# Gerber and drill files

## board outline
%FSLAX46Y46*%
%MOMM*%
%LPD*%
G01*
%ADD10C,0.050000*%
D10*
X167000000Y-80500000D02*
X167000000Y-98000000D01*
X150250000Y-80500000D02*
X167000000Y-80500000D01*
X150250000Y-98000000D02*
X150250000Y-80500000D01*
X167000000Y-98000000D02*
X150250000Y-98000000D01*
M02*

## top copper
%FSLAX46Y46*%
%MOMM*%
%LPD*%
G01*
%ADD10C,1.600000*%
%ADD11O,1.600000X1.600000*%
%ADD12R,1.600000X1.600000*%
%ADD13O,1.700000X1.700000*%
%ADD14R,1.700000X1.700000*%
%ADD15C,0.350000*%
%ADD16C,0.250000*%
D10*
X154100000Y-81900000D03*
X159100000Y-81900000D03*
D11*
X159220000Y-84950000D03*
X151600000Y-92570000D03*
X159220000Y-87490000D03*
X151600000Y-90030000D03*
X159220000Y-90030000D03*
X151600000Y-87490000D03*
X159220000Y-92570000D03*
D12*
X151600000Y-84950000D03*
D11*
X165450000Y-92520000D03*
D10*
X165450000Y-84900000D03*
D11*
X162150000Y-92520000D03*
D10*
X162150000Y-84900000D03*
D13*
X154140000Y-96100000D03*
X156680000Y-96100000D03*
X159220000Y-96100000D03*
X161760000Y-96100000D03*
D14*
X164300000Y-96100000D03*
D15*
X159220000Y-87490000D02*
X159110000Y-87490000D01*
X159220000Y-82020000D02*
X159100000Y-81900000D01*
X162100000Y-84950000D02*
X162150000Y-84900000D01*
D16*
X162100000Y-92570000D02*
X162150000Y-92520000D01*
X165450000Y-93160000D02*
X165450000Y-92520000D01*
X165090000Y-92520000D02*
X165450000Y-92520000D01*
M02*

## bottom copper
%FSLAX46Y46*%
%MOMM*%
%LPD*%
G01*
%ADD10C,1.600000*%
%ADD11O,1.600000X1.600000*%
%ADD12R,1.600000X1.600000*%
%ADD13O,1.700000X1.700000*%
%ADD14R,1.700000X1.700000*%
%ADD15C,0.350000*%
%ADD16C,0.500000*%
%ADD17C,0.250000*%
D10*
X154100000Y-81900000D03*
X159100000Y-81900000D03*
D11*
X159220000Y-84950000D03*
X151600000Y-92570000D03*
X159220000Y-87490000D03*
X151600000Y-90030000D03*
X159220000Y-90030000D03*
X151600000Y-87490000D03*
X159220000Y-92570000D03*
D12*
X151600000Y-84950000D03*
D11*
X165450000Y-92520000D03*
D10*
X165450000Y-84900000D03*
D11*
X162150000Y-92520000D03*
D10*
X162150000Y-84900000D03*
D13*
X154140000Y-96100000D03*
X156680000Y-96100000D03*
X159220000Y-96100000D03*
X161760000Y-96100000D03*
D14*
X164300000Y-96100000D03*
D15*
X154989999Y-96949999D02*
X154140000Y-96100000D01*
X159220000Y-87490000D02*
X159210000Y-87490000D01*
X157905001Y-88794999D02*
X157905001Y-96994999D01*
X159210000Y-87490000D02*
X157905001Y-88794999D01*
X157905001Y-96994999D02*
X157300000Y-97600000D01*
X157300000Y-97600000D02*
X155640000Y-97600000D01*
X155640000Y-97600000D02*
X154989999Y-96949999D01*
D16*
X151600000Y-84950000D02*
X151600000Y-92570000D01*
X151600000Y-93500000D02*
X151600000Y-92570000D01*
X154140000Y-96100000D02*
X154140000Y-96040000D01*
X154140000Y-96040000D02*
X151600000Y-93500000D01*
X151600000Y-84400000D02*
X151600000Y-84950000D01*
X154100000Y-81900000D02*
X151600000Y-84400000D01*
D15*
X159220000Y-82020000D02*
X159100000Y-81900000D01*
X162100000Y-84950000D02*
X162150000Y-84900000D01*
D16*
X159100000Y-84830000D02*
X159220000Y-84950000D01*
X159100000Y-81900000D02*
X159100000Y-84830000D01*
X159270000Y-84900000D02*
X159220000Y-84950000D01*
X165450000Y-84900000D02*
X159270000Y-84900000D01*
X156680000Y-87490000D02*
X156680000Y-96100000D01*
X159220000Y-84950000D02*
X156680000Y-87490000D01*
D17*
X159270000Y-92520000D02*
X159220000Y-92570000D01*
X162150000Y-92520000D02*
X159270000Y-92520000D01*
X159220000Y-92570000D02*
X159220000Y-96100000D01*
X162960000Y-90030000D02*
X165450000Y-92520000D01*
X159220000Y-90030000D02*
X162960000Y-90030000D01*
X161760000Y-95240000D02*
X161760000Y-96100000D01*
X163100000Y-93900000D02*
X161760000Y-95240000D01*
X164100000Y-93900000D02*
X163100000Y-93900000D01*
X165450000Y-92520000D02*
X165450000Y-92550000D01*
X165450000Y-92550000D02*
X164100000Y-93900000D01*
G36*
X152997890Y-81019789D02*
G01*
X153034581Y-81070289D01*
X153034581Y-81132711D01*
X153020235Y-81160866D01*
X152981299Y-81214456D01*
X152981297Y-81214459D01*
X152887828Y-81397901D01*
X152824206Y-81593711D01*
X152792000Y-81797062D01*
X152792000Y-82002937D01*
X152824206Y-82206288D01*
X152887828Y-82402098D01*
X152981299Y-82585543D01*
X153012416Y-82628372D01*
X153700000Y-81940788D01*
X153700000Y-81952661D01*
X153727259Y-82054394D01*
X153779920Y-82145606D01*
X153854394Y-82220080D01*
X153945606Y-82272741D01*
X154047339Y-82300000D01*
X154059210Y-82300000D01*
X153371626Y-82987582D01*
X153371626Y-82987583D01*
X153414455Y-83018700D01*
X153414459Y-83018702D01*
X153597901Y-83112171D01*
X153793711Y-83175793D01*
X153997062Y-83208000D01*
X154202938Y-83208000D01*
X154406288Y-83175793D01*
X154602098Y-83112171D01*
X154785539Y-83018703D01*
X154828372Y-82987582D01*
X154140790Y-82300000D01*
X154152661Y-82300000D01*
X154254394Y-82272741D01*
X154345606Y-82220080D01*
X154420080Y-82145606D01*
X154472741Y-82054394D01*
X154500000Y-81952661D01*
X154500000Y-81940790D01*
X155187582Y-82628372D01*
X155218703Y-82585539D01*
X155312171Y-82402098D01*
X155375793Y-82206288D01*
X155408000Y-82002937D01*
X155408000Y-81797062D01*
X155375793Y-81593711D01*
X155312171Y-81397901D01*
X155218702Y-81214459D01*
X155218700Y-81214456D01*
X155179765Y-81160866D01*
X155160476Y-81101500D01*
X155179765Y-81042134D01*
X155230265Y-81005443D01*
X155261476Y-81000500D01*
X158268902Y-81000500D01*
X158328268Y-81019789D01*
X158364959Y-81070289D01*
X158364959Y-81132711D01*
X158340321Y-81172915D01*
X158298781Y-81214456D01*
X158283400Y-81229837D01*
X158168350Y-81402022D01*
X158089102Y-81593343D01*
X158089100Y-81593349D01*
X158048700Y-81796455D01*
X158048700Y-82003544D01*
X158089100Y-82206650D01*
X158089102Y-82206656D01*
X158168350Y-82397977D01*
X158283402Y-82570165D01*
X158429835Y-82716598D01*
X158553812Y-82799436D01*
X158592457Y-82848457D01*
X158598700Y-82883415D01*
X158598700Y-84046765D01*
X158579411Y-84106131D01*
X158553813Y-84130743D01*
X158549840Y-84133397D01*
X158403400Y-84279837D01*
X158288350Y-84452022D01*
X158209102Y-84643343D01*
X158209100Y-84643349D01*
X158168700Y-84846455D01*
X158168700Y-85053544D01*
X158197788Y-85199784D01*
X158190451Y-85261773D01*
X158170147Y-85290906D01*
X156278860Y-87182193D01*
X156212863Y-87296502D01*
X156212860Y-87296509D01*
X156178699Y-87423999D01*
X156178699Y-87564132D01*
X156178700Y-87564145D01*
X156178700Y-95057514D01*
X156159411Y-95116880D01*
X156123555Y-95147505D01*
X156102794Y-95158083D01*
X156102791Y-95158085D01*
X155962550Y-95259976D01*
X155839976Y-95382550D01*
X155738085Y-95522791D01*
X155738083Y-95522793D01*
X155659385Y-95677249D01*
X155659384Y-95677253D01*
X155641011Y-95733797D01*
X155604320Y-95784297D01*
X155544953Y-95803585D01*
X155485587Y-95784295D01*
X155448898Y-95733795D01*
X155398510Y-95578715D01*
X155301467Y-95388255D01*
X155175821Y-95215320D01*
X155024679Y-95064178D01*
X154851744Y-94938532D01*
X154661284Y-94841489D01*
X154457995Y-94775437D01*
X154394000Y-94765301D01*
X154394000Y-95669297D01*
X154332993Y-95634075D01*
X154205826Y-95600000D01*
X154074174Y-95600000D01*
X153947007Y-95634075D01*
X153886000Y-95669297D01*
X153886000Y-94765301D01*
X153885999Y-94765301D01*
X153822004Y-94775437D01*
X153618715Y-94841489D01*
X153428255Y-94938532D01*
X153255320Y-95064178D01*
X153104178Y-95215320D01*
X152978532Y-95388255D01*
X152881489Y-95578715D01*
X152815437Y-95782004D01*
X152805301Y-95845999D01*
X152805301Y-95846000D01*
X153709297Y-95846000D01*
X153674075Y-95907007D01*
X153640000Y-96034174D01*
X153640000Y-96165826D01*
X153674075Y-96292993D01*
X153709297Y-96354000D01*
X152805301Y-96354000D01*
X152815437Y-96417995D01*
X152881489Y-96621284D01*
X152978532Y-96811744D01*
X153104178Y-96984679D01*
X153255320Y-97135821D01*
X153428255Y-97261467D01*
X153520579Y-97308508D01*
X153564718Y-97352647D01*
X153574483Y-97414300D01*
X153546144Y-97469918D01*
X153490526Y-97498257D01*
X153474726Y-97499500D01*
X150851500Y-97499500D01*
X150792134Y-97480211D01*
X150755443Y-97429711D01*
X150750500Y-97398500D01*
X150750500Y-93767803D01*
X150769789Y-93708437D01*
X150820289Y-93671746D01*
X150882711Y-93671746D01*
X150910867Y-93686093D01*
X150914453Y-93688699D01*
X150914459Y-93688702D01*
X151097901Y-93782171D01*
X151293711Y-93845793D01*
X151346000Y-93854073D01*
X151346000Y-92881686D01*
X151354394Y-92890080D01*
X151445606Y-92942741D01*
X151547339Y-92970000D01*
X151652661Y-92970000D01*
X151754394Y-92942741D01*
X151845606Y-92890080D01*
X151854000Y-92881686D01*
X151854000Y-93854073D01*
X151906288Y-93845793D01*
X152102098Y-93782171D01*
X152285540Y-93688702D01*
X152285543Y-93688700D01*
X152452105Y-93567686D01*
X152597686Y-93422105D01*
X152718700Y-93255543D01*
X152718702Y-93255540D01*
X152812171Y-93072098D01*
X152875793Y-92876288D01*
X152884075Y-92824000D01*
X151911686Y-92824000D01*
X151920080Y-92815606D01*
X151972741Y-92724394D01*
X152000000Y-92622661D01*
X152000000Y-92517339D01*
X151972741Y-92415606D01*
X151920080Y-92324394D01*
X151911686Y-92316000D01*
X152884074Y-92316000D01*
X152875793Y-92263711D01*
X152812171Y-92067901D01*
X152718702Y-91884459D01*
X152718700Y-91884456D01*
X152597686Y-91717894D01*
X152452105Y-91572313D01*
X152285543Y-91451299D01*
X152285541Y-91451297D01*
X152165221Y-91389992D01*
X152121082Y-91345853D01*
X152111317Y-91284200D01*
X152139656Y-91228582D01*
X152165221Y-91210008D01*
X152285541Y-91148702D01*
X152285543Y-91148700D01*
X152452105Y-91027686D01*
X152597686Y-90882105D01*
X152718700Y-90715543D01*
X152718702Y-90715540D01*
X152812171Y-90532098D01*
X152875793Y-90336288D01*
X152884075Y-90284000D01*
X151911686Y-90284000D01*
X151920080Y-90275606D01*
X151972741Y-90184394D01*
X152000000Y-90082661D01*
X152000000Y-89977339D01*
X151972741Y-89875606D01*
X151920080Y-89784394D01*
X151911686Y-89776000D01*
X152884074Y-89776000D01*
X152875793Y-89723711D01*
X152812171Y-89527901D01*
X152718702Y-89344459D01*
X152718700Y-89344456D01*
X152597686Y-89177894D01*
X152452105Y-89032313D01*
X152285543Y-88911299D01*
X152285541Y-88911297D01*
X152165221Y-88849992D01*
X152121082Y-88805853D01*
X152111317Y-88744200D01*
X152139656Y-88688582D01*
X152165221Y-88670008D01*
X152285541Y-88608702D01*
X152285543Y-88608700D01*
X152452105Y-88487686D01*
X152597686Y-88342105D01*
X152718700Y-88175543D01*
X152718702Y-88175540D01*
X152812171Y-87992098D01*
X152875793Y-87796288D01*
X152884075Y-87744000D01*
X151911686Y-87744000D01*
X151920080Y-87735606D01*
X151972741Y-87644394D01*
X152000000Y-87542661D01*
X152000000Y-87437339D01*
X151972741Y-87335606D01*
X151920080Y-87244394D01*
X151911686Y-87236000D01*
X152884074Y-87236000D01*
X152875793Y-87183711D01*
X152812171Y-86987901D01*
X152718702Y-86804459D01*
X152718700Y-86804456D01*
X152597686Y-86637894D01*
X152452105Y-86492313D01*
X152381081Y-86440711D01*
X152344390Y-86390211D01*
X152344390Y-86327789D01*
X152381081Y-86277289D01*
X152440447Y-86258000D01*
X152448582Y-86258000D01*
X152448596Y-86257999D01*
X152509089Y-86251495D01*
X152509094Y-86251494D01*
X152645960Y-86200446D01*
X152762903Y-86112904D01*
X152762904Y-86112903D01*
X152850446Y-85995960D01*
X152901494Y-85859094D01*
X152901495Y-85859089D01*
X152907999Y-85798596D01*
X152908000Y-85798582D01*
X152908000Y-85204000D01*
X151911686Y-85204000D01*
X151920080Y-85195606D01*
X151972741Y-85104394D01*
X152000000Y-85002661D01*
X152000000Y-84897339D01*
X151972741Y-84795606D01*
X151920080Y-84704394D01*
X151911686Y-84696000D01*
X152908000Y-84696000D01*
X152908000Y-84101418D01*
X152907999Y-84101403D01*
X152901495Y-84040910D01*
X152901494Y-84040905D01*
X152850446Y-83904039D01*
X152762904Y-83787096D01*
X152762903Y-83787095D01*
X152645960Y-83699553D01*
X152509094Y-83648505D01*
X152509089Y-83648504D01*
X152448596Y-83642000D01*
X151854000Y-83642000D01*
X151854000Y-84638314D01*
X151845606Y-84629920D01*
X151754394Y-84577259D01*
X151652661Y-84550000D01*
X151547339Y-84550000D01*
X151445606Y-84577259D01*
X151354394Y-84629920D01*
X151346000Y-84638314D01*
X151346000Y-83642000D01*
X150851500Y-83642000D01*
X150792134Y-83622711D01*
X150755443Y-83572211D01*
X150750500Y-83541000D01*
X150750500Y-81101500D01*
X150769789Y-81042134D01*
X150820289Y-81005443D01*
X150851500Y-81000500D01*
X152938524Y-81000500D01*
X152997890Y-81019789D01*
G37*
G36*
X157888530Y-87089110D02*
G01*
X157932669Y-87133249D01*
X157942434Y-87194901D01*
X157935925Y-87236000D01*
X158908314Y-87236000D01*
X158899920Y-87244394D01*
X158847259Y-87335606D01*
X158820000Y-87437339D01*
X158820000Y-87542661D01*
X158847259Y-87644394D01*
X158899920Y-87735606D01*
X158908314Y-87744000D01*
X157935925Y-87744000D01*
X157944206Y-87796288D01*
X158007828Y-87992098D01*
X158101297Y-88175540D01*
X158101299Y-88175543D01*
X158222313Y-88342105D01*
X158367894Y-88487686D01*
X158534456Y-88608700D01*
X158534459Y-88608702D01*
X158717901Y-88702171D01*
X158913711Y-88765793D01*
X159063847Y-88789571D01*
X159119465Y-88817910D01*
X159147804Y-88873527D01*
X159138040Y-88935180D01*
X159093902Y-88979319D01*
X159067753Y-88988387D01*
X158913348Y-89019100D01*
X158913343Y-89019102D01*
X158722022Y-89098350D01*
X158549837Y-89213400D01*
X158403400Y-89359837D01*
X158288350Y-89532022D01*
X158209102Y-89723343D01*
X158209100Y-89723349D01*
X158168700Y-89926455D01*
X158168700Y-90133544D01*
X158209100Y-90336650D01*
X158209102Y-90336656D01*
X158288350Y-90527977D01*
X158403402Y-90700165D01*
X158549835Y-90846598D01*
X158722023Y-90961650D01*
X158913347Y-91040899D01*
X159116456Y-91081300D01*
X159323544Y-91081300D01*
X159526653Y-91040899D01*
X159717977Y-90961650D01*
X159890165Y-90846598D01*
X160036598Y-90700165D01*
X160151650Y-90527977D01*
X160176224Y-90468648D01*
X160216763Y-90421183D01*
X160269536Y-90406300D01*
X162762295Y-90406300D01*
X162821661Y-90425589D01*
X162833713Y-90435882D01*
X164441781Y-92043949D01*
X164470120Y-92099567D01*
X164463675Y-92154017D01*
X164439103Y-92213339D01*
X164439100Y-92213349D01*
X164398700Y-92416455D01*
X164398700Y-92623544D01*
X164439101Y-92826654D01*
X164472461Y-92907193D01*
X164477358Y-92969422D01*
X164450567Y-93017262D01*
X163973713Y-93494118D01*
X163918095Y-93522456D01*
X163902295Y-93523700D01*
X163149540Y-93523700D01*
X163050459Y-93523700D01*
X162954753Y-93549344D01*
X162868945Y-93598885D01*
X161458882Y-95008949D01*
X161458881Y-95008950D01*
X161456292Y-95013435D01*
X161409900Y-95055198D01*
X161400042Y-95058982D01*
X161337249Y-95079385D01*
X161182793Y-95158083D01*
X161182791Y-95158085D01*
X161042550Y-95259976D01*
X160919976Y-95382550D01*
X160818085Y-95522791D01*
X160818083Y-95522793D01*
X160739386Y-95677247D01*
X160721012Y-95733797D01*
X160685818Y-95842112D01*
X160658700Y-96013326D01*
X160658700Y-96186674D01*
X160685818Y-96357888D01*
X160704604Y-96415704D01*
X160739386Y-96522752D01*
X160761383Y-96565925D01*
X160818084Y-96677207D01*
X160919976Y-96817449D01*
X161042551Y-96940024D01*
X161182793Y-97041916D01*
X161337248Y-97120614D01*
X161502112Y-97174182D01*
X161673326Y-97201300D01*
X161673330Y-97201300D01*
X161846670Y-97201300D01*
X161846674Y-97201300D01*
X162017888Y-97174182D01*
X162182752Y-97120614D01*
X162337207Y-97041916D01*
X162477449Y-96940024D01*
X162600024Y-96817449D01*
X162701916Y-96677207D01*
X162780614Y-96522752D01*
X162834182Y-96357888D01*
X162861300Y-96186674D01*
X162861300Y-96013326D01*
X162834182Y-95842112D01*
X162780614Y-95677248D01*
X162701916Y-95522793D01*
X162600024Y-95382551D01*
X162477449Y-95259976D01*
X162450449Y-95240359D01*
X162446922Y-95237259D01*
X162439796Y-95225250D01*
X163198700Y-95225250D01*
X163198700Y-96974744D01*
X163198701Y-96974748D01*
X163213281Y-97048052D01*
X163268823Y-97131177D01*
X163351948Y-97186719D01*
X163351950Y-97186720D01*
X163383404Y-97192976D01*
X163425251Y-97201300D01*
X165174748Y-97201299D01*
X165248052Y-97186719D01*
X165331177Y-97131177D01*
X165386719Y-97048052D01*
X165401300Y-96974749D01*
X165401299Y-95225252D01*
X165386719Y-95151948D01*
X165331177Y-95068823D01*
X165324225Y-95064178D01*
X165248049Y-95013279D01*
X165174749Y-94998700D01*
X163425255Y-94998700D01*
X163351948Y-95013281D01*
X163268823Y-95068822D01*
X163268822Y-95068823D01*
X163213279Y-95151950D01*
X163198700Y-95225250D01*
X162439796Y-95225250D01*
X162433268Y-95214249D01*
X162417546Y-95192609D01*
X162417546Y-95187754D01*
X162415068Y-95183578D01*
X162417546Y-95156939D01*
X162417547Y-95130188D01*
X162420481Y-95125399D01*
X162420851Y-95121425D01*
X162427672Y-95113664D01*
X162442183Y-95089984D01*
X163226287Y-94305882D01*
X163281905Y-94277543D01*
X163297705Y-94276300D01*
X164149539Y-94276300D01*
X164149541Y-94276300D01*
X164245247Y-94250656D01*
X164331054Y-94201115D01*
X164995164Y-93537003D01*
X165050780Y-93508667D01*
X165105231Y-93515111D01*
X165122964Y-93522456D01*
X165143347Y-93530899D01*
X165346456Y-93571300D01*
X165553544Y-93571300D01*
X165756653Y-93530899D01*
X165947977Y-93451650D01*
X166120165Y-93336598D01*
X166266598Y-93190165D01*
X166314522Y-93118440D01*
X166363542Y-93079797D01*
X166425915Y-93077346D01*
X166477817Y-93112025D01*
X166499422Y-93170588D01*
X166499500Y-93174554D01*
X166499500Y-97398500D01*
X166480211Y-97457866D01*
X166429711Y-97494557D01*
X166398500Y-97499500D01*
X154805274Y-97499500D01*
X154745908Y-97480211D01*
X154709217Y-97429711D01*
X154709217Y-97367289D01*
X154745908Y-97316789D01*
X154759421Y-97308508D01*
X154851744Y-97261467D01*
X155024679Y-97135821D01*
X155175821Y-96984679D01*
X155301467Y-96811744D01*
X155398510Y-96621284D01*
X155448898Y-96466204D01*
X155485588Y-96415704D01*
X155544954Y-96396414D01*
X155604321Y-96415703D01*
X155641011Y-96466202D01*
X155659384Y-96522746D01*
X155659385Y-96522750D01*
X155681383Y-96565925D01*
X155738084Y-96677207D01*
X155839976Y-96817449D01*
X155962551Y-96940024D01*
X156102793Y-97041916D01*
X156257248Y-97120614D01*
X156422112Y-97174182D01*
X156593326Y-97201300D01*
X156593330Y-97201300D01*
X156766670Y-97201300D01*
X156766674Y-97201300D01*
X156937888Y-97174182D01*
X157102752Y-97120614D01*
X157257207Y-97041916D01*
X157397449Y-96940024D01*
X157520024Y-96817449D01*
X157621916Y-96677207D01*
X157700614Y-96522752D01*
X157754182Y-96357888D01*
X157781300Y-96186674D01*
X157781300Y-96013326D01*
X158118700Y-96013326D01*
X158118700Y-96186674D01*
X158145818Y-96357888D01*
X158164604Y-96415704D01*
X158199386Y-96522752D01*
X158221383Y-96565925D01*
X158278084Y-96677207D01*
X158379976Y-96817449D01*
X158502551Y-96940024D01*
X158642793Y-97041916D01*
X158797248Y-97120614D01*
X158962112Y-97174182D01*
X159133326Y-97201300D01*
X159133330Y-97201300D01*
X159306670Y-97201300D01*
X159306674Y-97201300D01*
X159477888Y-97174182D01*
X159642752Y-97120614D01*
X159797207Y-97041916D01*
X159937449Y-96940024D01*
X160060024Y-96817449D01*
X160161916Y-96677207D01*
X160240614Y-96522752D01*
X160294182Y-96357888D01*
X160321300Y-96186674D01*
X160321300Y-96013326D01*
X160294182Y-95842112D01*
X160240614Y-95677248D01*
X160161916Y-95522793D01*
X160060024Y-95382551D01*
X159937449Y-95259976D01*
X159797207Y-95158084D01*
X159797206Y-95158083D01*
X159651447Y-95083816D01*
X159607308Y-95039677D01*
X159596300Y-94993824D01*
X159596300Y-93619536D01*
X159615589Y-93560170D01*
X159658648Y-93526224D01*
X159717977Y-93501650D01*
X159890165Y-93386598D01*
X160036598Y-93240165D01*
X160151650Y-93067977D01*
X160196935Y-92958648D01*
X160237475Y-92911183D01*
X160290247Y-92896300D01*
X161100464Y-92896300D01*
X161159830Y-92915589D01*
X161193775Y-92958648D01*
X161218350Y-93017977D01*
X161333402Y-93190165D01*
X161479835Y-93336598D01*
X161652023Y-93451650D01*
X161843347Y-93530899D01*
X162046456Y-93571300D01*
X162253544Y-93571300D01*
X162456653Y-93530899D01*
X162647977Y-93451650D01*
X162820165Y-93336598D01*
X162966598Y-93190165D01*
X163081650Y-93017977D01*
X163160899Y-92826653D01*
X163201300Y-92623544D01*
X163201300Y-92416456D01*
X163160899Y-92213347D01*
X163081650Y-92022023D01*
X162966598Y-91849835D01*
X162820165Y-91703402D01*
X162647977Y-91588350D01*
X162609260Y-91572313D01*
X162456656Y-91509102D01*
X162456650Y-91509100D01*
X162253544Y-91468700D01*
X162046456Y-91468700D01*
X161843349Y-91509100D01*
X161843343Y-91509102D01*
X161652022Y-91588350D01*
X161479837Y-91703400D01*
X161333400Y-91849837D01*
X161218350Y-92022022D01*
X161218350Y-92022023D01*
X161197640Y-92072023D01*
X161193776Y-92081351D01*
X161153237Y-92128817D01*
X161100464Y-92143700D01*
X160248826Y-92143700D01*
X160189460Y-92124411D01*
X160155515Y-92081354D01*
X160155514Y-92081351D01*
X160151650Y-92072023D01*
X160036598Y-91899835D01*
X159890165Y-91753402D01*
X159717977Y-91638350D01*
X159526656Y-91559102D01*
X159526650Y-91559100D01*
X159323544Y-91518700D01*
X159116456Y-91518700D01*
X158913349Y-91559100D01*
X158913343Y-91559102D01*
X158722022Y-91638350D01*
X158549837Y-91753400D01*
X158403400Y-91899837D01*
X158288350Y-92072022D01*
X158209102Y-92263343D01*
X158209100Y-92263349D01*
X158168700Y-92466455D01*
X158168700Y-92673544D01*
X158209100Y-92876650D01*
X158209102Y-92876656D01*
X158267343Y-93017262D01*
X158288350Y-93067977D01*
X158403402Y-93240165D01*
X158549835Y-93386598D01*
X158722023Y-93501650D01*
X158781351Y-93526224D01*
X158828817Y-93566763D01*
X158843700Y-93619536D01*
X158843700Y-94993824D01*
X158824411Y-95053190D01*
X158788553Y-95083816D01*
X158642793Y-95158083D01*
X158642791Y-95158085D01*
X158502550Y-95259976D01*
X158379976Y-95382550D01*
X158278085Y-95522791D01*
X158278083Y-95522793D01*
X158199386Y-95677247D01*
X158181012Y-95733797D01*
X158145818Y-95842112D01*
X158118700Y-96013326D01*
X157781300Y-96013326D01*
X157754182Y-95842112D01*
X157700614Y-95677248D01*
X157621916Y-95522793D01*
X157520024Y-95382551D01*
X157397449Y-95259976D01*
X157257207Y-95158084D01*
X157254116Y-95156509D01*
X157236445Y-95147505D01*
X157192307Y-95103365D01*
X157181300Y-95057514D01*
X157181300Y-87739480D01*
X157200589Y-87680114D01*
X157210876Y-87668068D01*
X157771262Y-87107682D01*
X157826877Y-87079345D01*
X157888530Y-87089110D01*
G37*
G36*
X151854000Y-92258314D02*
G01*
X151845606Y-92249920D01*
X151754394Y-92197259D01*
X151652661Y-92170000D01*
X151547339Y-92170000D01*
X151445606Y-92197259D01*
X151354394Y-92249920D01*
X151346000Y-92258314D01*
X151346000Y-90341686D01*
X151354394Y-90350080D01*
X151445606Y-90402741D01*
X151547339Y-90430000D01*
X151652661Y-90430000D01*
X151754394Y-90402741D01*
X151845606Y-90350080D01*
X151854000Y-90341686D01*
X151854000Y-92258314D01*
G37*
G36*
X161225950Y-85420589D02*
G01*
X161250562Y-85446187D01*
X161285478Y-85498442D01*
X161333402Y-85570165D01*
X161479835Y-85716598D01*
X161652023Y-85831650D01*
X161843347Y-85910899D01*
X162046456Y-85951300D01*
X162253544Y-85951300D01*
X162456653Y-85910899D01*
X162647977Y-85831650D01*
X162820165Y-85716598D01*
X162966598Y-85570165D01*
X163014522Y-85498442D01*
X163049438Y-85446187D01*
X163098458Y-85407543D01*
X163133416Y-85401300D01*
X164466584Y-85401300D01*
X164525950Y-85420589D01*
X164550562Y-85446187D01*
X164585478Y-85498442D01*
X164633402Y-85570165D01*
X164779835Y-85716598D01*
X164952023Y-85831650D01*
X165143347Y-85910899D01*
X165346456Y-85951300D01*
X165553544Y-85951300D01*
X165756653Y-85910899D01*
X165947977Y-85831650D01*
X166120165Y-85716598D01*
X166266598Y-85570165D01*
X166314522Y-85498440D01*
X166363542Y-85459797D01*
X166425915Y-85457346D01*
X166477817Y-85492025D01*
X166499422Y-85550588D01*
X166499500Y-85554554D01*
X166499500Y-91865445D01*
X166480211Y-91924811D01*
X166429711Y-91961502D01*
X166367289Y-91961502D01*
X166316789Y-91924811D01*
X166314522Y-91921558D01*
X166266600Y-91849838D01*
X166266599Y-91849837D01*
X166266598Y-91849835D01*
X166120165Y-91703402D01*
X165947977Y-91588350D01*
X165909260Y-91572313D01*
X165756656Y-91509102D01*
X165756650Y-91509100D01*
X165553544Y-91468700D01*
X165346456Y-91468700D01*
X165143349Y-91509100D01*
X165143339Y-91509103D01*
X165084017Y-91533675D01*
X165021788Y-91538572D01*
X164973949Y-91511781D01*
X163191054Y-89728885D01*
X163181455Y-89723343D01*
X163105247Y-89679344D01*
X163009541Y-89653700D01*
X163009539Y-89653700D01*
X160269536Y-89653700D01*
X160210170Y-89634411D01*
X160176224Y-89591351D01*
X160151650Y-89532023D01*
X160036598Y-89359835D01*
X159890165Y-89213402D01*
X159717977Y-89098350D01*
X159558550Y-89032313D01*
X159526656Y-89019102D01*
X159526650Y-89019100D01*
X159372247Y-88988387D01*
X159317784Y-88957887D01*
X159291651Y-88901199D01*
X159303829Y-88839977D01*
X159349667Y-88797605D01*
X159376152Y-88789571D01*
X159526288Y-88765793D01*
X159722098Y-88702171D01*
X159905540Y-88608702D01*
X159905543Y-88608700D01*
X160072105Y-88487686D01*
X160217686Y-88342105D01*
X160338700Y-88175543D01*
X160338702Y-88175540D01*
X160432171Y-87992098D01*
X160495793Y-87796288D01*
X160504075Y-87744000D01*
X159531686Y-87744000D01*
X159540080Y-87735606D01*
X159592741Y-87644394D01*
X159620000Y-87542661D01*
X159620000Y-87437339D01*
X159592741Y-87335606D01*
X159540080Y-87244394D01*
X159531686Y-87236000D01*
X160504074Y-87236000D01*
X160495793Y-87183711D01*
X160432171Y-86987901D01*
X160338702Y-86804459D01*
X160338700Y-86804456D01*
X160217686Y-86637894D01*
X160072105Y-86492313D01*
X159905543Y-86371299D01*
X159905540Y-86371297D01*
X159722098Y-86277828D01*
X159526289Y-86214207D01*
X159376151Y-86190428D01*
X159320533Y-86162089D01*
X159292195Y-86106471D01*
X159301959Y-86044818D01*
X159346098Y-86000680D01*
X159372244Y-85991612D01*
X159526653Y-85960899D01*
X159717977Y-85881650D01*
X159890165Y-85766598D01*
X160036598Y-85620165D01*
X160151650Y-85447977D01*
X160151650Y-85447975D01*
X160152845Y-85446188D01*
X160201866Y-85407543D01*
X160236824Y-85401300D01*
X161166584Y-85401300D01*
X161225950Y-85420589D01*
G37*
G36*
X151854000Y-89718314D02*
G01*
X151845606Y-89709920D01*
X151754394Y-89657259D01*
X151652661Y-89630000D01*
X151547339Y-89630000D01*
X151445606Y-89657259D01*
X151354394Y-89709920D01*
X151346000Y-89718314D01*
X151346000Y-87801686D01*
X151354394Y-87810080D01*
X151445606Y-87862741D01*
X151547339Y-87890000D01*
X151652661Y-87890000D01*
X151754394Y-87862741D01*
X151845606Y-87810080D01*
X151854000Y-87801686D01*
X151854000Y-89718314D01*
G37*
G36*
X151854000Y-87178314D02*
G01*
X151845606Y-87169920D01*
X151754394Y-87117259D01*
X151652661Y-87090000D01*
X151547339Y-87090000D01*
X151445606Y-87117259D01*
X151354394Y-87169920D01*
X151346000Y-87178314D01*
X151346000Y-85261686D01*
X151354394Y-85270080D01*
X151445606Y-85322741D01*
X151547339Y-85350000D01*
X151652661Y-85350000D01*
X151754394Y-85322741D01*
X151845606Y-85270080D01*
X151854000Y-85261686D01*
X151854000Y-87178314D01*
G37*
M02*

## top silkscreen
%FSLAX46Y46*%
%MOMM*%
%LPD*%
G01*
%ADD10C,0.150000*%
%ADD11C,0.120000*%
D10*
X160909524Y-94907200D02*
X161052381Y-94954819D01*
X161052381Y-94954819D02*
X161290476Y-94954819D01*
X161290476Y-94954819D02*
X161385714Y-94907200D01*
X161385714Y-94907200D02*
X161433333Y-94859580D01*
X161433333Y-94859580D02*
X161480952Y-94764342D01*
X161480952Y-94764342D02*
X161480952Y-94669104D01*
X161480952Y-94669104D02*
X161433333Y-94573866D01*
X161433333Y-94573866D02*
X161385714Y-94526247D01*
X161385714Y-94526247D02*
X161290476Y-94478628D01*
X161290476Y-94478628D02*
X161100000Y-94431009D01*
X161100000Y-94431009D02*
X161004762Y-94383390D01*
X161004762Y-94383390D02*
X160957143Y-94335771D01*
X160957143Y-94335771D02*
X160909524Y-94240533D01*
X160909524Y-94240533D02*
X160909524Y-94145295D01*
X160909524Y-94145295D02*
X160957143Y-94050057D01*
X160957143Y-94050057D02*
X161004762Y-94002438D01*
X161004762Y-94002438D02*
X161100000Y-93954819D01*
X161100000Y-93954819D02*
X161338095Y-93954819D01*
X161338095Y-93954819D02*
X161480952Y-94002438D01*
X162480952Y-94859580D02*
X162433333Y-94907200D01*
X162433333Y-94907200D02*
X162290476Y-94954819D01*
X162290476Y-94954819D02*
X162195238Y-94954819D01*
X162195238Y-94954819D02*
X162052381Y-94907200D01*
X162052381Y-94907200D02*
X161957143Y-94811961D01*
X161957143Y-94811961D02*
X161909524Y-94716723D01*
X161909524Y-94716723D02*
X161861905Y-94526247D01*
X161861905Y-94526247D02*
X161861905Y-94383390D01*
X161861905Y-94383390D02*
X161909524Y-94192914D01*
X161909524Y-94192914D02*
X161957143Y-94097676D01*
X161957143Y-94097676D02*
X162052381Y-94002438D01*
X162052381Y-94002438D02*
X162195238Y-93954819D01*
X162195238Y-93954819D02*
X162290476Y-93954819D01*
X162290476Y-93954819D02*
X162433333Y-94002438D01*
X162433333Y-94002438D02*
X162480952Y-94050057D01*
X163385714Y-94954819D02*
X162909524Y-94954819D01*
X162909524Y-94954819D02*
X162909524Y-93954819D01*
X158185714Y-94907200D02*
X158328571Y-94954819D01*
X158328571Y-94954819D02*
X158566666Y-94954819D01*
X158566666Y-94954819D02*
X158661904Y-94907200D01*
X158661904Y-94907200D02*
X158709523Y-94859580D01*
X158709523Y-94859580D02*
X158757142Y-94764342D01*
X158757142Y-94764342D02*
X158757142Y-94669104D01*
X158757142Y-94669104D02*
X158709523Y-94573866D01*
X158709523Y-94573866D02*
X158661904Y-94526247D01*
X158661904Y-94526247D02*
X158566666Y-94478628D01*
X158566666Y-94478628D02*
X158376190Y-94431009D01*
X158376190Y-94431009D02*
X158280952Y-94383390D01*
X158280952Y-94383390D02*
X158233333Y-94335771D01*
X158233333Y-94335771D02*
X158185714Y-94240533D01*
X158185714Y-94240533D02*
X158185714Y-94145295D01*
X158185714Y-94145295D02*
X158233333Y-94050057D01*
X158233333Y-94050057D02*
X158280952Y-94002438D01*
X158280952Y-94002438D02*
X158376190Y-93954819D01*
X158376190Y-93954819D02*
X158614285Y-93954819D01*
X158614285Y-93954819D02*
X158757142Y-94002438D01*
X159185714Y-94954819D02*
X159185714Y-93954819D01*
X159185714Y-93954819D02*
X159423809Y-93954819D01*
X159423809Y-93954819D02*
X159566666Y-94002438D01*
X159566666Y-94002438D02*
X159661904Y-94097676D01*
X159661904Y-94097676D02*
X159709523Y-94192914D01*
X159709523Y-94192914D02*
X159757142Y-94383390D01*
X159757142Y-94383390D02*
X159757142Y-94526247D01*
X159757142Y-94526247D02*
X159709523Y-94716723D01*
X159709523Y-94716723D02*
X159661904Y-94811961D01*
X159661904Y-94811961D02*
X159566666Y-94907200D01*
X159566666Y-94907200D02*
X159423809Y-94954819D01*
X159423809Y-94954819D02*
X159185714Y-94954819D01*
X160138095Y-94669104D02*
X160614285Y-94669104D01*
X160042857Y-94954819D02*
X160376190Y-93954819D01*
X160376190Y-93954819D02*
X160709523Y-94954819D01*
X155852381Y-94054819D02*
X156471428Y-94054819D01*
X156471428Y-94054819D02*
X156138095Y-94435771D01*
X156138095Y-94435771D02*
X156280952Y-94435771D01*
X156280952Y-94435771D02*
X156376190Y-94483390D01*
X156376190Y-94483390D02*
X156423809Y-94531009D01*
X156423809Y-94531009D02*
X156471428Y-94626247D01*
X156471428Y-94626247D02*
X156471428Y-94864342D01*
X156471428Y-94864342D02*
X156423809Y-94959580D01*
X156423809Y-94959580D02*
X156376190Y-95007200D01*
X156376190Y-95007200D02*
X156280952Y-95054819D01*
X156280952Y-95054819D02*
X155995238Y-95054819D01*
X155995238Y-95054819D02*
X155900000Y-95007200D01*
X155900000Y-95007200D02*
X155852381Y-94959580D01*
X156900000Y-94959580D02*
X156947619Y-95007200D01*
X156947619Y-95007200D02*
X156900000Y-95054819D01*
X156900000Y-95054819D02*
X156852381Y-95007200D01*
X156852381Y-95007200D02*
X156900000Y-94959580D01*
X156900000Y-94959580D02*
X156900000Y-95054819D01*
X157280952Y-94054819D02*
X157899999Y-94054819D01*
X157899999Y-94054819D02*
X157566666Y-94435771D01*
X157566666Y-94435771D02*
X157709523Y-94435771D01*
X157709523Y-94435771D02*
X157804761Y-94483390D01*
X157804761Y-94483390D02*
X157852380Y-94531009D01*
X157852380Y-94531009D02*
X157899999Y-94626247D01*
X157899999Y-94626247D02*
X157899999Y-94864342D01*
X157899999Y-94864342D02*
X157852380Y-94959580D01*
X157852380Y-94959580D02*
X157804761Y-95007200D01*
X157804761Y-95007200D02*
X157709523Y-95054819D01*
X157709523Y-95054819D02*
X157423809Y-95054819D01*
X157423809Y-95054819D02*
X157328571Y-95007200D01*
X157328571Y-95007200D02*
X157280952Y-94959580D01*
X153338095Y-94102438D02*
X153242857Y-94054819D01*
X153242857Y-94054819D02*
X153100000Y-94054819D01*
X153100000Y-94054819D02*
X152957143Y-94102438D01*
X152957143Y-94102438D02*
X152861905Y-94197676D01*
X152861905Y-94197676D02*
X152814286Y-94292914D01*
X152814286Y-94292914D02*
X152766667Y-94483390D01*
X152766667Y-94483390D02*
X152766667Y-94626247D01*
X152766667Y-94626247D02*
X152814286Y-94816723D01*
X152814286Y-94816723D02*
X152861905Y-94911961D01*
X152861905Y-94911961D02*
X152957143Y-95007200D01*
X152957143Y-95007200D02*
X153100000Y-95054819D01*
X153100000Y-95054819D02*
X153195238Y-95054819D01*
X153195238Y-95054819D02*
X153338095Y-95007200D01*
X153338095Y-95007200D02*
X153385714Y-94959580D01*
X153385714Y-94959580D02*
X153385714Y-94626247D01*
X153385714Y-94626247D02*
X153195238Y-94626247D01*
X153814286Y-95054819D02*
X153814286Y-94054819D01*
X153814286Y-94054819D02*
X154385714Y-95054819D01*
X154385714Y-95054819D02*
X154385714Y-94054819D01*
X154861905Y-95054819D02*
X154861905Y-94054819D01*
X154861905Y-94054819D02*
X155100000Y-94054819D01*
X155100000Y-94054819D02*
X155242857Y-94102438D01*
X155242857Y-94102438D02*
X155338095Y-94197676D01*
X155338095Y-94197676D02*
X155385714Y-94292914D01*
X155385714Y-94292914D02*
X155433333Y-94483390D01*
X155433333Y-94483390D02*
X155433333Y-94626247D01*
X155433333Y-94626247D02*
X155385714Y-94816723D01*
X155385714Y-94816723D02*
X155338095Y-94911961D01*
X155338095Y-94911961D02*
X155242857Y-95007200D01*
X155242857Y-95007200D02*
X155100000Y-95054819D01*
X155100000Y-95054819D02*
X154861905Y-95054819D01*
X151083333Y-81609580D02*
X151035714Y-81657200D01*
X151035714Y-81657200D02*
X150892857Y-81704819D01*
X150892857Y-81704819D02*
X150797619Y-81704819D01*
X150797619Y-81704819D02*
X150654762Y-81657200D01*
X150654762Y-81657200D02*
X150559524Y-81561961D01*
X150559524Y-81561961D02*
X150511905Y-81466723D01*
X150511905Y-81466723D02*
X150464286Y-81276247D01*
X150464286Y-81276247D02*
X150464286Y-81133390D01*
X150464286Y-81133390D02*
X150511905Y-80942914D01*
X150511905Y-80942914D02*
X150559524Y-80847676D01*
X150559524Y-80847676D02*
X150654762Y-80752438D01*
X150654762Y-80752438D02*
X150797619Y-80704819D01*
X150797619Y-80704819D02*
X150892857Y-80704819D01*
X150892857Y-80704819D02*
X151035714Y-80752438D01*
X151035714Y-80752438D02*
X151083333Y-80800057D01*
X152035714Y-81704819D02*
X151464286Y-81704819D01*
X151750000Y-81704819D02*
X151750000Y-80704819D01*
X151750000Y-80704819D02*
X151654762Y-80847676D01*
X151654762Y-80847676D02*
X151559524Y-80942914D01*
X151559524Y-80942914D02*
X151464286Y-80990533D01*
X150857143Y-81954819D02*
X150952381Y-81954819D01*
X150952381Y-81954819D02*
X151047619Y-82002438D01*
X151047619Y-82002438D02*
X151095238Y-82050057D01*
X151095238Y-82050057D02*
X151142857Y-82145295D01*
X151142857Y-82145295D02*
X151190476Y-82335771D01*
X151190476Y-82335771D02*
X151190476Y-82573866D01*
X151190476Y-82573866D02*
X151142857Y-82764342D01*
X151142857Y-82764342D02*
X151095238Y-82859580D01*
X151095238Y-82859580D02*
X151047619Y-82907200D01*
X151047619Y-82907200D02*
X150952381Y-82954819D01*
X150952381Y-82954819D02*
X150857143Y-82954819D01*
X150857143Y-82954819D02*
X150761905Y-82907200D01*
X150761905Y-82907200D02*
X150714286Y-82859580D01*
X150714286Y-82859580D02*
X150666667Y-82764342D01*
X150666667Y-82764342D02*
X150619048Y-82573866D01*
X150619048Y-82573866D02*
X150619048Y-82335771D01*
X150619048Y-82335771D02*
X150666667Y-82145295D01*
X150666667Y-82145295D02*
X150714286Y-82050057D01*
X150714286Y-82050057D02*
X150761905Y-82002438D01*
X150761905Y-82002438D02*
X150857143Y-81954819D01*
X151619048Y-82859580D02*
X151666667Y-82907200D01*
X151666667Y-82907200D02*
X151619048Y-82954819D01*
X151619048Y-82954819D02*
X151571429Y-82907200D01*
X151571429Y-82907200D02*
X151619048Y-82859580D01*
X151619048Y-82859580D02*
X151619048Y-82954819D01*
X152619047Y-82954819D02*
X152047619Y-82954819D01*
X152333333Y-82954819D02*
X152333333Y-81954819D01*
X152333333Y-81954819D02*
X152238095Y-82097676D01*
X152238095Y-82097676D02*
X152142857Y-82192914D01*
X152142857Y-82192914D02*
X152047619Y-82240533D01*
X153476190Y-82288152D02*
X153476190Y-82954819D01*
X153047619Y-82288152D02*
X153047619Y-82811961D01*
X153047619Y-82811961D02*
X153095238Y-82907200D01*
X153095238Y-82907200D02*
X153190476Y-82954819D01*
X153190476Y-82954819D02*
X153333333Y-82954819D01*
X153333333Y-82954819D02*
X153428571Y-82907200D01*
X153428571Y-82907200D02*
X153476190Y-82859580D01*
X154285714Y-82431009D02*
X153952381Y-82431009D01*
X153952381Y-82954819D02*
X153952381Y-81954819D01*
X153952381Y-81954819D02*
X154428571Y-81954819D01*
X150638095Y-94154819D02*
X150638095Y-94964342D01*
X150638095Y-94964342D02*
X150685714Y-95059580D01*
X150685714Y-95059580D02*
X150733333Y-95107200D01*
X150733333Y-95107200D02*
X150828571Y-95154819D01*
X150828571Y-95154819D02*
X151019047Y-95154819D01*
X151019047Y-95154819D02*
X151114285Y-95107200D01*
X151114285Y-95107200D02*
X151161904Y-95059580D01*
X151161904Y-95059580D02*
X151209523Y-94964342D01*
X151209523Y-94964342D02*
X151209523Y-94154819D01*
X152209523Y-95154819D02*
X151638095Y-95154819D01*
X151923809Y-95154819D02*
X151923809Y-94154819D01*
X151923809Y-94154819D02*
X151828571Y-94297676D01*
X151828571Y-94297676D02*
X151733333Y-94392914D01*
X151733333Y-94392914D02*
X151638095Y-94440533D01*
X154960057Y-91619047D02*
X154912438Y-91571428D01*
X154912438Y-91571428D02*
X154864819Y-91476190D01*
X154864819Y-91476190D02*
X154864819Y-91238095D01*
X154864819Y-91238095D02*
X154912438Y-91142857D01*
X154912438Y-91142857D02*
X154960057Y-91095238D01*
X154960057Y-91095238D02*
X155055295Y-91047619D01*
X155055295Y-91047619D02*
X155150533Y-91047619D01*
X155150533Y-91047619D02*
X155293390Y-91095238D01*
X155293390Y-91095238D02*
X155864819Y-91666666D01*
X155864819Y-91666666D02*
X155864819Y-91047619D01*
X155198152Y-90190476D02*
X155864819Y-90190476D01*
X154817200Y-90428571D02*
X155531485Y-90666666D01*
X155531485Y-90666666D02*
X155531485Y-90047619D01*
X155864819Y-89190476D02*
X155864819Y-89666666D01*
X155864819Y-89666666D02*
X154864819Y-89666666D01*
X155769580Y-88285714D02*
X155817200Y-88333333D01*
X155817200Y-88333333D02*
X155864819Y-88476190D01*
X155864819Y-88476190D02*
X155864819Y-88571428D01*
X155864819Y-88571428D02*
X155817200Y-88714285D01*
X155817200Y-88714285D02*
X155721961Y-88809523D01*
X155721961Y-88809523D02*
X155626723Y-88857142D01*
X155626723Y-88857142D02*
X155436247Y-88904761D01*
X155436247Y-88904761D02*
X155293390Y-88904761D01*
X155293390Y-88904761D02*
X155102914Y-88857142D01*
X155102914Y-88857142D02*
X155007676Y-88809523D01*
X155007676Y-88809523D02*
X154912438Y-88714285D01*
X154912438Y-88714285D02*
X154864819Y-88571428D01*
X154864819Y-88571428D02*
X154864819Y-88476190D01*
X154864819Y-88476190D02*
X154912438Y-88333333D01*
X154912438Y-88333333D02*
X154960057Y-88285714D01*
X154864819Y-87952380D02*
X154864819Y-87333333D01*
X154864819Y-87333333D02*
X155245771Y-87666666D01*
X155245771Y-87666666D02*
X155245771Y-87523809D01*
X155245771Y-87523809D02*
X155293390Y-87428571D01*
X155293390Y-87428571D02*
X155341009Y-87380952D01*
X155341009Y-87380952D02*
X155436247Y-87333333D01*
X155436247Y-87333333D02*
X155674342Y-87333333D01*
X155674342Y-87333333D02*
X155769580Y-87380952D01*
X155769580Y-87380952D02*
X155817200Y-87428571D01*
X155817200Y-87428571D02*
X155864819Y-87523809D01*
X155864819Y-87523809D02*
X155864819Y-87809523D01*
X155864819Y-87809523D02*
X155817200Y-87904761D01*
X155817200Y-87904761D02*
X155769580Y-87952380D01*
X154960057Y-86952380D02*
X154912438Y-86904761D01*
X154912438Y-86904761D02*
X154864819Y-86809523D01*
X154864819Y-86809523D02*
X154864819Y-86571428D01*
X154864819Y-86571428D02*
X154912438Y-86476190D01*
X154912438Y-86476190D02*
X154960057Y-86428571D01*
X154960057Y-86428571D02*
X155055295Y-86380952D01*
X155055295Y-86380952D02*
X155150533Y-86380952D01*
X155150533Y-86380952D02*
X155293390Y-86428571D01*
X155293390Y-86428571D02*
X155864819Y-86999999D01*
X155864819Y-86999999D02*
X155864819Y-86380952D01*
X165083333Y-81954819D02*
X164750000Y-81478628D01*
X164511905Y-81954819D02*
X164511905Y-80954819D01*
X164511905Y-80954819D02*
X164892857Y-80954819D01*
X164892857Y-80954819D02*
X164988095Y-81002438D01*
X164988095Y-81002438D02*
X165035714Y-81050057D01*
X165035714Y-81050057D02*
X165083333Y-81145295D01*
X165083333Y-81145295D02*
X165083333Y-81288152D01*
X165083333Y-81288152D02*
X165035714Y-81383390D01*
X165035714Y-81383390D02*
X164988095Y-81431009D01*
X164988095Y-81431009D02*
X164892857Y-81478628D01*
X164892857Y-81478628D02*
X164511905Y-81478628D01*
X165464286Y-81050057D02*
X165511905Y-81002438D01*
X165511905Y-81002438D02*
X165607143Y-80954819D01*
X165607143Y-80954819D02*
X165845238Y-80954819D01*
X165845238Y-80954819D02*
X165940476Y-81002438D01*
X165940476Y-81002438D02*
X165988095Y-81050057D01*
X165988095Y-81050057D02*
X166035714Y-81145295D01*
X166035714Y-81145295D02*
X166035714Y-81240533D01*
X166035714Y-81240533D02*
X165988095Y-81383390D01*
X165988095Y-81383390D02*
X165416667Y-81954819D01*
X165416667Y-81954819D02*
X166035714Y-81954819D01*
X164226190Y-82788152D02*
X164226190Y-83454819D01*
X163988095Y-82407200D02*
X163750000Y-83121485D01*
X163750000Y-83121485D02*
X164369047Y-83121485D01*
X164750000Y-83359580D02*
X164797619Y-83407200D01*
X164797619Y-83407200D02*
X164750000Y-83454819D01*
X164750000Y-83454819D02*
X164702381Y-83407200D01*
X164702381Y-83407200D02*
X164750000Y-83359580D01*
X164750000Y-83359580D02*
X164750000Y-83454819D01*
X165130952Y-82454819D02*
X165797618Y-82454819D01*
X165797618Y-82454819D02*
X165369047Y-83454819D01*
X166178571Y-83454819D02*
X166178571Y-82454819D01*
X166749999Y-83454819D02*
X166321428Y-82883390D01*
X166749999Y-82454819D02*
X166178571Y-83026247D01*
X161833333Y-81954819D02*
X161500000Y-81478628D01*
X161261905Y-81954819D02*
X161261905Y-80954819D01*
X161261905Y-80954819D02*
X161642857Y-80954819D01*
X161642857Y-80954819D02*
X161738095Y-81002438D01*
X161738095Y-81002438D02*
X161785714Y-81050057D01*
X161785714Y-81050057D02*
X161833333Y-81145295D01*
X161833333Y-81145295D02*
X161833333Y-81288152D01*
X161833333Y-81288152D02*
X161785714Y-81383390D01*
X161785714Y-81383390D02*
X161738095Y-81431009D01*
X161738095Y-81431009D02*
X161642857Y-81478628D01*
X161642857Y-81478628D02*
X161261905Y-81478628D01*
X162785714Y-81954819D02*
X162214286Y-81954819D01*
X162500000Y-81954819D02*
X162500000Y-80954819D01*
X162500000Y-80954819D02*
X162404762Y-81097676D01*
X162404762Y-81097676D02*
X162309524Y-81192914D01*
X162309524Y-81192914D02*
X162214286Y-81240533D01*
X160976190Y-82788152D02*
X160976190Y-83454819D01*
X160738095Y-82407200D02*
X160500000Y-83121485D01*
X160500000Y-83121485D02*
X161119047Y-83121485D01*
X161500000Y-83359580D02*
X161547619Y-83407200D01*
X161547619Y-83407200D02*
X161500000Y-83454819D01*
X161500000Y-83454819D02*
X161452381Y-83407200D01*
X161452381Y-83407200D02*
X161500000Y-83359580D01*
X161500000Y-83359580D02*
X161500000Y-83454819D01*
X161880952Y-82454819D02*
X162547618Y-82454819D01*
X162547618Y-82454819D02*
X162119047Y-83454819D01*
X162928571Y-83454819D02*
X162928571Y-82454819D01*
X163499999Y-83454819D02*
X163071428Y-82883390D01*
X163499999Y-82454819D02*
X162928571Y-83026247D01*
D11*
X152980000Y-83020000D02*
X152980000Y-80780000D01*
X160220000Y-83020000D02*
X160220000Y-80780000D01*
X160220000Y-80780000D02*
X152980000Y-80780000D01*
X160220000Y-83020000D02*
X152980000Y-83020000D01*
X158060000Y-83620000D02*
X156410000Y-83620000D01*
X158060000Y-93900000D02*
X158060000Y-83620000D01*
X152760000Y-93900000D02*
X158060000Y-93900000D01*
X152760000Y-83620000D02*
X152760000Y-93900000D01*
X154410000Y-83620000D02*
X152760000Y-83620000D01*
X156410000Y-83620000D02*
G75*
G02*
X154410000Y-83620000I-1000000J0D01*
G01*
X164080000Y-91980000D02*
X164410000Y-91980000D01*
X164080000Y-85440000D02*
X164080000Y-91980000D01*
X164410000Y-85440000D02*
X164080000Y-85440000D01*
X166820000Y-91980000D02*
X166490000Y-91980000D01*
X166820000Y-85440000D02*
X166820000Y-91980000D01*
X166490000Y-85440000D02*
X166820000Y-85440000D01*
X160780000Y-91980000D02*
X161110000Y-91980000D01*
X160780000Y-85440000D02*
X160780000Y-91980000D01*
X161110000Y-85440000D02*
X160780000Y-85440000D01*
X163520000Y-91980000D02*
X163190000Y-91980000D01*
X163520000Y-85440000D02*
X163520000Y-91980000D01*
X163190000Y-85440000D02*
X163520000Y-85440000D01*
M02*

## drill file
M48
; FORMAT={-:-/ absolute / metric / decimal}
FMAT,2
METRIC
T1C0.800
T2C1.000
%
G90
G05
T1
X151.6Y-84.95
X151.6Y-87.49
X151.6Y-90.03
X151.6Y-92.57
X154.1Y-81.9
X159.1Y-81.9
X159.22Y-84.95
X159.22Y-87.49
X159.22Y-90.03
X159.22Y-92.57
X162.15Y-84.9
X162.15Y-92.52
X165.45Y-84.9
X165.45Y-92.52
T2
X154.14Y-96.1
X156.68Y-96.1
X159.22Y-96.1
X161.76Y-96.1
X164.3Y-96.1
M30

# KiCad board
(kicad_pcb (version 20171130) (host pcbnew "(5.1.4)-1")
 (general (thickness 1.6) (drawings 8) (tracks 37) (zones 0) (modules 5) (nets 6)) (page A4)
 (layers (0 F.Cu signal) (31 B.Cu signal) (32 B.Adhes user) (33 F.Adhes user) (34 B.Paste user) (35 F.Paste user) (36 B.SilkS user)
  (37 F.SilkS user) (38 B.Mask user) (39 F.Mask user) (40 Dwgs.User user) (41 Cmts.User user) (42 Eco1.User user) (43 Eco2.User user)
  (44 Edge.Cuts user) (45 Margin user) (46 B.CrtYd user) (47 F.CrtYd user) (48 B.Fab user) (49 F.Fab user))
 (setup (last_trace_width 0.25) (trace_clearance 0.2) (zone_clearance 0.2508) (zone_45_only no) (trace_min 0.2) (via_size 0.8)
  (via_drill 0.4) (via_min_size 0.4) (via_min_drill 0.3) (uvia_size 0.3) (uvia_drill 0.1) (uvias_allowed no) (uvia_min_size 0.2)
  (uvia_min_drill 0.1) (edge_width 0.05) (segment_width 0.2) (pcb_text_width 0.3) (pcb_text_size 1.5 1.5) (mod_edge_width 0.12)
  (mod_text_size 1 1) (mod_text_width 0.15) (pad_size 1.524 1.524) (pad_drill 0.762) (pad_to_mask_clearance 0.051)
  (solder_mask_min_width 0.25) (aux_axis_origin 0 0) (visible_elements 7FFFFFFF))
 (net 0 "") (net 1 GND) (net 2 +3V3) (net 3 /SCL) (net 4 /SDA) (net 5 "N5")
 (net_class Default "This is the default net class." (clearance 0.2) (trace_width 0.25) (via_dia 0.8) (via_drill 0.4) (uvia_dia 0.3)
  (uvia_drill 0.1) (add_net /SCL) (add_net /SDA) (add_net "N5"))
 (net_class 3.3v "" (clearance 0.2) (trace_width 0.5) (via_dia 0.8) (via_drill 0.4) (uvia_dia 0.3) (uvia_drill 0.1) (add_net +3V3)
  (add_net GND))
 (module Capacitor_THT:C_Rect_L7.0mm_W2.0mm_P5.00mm (layer F.Cu) (at 159.1 81.9 180)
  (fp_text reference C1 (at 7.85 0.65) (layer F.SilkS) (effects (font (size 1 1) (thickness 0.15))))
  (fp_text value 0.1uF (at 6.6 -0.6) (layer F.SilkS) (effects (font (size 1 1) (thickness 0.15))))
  (fp_line (start 6.12 -1.12) (end 6.12 1.12) (layer F.SilkS) (width 0.12))
  (fp_line (start -1.12 -1.12) (end -1.12 1.12) (layer F.SilkS) (width 0.12))
  (fp_line (start -1.12 1.12) (end 6.12 1.12) (layer F.SilkS) (width 0.12))
  (fp_line (start -1.12 -1.12) (end 6.12 -1.12) (layer F.SilkS) (width 0.12))
  (pad 2 thru_hole circle (at 5 0 180) (size 1.6 1.6) (drill 0.8) (layers *.Cu *.Mask) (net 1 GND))
  (pad 1 thru_hole circle (at 0 0 180) (size 1.6 1.6) (drill 0.8) (layers *.Cu *.Mask) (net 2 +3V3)))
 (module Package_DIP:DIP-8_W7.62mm (layer F.Cu) (at 151.6 84.95)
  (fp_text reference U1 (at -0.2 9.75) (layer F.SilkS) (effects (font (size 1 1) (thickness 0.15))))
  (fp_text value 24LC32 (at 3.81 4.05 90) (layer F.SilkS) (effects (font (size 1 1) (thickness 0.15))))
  (fp_line (start 6.46 -1.33) (end 4.81 -1.33) (layer F.SilkS) (width 0.12))
  (fp_line (start 6.46 8.95) (end 6.46 -1.33) (layer F.SilkS) (width 0.12))
  (fp_line (start 1.16 8.95) (end 6.46 8.95) (layer F.SilkS) (width 0.12))
  (fp_line (start 1.16 -1.33) (end 1.16 8.95) (layer F.SilkS) (width 0.12))
  (fp_line (start 2.81 -1.33) (end 1.16 -1.33) (layer F.SilkS) (width 0.12))
  (fp_arc (start 3.81 -1.33) (end 2.81 -1.33) (angle -180) (layer F.SilkS) (width 0.12))
  (pad 8 thru_hole oval (at 7.62 0) (size 1.6 1.6) (drill 0.8) (layers *.Cu *.Mask) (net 2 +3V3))
  (pad 4 thru_hole oval (at 0 7.62) (size 1.6 1.6) (drill 0.8) (layers *.Cu *.Mask) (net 1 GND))
  (pad 7 thru_hole oval (at 7.62 2.54) (size 1.6 1.6) (drill 0.8) (layers *.Cu *.Mask) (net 1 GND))
  (pad 3 thru_hole oval (at 0 5.08) (size 1.6 1.6) (drill 0.8) (layers *.Cu *.Mask) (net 1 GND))
  (pad 6 thru_hole oval (at 7.62 5.08) (size 1.6 1.6) (drill 0.8) (layers *.Cu *.Mask) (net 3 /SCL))
  (pad 2 thru_hole oval (at 0 2.54) (size 1.6 1.6) (drill 0.8) (layers *.Cu *.Mask) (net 1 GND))
  (pad 5 thru_hole oval (at 7.62 7.62) (size 1.6 1.6) (drill 0.8) (layers *.Cu *.Mask) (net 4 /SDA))
  (pad 1 thru_hole rect (at 0 0) (size 1.6 1.6) (drill 0.8) (layers *.Cu *.Mask) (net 1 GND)))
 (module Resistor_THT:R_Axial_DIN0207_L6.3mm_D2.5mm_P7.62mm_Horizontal (layer F.Cu) (at 165.45 84.9 270)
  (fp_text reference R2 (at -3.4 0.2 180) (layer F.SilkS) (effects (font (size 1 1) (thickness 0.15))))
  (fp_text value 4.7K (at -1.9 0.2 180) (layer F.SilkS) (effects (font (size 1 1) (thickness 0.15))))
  (fp_line (start 7.08 1.37) (end 7.08 1.04) (layer F.SilkS) (width 0.12))
  (fp_line (start 0.54 1.37) (end 7.08 1.37) (layer F.SilkS) (width 0.12))
  (fp_line (start 0.54 1.04) (end 0.54 1.37) (layer F.SilkS) (width 0.12))
  (fp_line (start 7.08 -1.37) (end 7.08 -1.04) (layer F.SilkS) (width 0.12))
  (fp_line (start 0.54 -1.37) (end 7.08 -1.37) (layer F.SilkS) (width 0.12))
  (fp_line (start 0.54 -1.04) (end 0.54 -1.37) (layer F.SilkS) (width 0.12))
  (pad 2 thru_hole oval (at 7.62 0 270) (size 1.6 1.6) (drill 0.8) (layers *.Cu *.Mask) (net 3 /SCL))
  (pad 1 thru_hole circle (at 0 0 270) (size 1.6 1.6) (drill 0.8) (layers *.Cu *.Mask) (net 2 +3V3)))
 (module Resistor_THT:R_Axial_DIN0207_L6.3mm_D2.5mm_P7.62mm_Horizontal (layer F.Cu) (at 162.15 84.9 270)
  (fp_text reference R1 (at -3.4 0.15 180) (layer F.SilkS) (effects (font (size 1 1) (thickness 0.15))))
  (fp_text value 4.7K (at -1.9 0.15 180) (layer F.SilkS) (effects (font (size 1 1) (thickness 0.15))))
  (fp_line (start 7.08 1.37) (end 7.08 1.04) (layer F.SilkS) (width 0.12))
  (fp_line (start 0.54 1.37) (end 7.08 1.37) (layer F.SilkS) (width 0.12))
  (fp_line (start 0.54 1.04) (end 0.54 1.37) (layer F.SilkS) (width 0.12))
  (fp_line (start 7.08 -1.37) (end 7.08 -1.04) (layer F.SilkS) (width 0.12))
  (fp_line (start 0.54 -1.37) (end 7.08 -1.37) (layer F.SilkS) (width 0.12))
  (fp_line (start 0.54 -1.04) (end 0.54 -1.37) (layer F.SilkS) (width 0.12))
  (pad 2 thru_hole oval (at 7.62 0 270) (size 1.6 1.6) (drill 0.8) (layers *.Cu *.Mask) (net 4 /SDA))
  (pad 1 thru_hole circle (at 0 0 270) (size 1.6 1.6) (drill 0.8) (layers *.Cu *.Mask) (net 2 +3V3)))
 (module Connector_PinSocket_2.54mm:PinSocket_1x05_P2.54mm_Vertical (layer B.Cu) (at 164.3 96.1 90)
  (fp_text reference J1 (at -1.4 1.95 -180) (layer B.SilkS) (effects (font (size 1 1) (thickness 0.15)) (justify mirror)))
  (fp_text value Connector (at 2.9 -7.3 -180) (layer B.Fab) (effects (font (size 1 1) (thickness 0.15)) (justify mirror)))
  (pad 5 thru_hole oval (at 0 -10.16 90) (size 1.7 1.7) (drill 1) (layers *.Cu *.Mask) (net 1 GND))
  (pad 4 thru_hole oval (at 0 -7.62 90) (size 1.7 1.7) (drill 1) (layers *.Cu *.Mask) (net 2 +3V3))
  (pad 3 thru_hole oval (at 0 -5.08 90) (size 1.7 1.7) (drill 1) (layers *.Cu *.Mask) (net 4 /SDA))
  (pad 2 thru_hole oval (at 0 -2.54 90) (size 1.7 1.7) (drill 1) (layers *.Cu *.Mask) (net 3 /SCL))
  (pad 1 thru_hole rect (at 0 0 90) (size 1.7 1.7) (drill 1) (layers *.Cu *.Mask) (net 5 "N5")))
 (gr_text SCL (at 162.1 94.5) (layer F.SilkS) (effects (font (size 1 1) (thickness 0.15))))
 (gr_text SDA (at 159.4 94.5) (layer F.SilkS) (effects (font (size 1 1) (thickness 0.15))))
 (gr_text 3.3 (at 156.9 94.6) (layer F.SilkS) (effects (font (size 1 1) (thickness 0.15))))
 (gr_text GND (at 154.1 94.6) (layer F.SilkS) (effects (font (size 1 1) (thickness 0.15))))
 (gr_line (start 167 80.5) (end 167 98) (layer Edge.Cuts) (width 0.05))
 (gr_line (start 150.25 80.5) (end 167 80.5) (layer Edge.Cuts) (width 0.05))
 (gr_line (start 150.25 98) (end 150.25 80.5) (layer Edge.Cuts) (width 0.05))
 (gr_line (start 167 98) (end 150.25 98) (layer Edge.Cuts) (width 0.05))
 (segment (start 159.22 87.49) (end 159.11 87.49) (width 0.35) (layer F.Cu) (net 1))
 (segment (start 154.989999 96.949999) (end 154.14 96.1) (width 0.35) (layer B.Cu) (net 1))
 (segment (start 159.22 87.49) (end 159.21 87.49) (width 0.35) (layer B.Cu) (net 1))
 (segment (start 157.905001 88.794999) (end 157.905001 96.994999) (width 0.35) (layer B.Cu) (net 1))
 (segment (start 159.21 87.49) (end 157.905001 88.794999) (width 0.35) (layer B.Cu) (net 1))
 (segment (start 157.905001 96.994999) (end 157.3 97.6) (width 0.35) (layer B.Cu) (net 1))
 (segment (start 157.3 97.6) (end 155.64 97.6) (width 0.35) (layer B.Cu) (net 1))
 (segment (start 155.64 97.6) (end 154.989999 96.949999) (width 0.35) (layer B.Cu) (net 1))
 (segment (start 151.6 84.95) (end 151.6 92.57) (width 0.5) (layer B.Cu) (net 1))
 (segment (start 151.6 93.5) (end 151.6 92.57) (width 0.5) (layer B.Cu) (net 1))
 (segment (start 154.14 96.1) (end 154.14 96.04) (width 0.5) (layer B.Cu) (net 1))
 (segment (start 154.14 96.04) (end 151.6 93.5) (width 0.5) (layer B.Cu) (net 1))
 (segment (start 151.6 84.4) (end 151.6 84.95) (width 0.5) (layer B.Cu) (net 1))
 (segment (start 154.1 81.9) (end 151.6 84.4) (width 0.5) (layer B.Cu) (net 1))
 (segment (start 159.22 82.02) (end 159.1 81.9) (width 0.35) (layer F.Cu) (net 2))
 (segment (start 162.1 84.95) (end 162.15 84.9) (width 0.35) (layer F.Cu) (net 2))
 (segment (start 159.22 82.02) (end 159.1 81.9) (width 0.35) (layer B.Cu) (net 2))
 (segment (start 162.1 84.95) (end 162.15 84.9) (width 0.35) (layer B.Cu) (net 2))
 (segment (start 159.1 84.83) (end 159.22 84.95) (width 0.5) (layer B.Cu) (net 2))
 (segment (start 159.1 81.9) (end 159.1 84.83) (width 0.5) (layer B.Cu) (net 2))
 (segment (start 159.27 84.9) (end 159.22 84.95) (width 0.5) (layer B.Cu) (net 2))
 (segment (start 165.45 84.9) (end 159.27 84.9) (width 0.5) (layer B.Cu) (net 2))
 (segment (start 156.68 87.49) (end 156.68 96.1) (width 0.5) (layer B.Cu) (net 2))
 (segment (start 159.22 84.95) (end 156.68 87.49) (width 0.5) (layer B.Cu) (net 2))
 (segment (start 162.1 92.57) (end 162.15 92.52) (width 0.25) (layer F.Cu) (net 4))
 (segment (start 159.27 92.52) (end 159.22 92.57) (width 0.25) (layer B.Cu) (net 4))
 (segment (start 162.15 92.52) (end 159.27 92.52) (width 0.25) (layer B.Cu) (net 4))
 (segment (start 159.22 92.57) (end 159.22 96.1) (width 0.25) (layer B.Cu) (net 4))
 (segment (start 165.45 93.16) (end 165.45 92.52) (width 0.25) (layer F.Cu) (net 3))
 (segment (start 165.09 92.52) (end 165.45 92.52) (width 0.25) (layer F.Cu) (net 3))
 (segment (start 162.96 90.03) (end 165.45 92.52) (width 0.25) (layer B.Cu) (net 3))
 (segment (start 159.22 90.03) (end 162.96 90.03) (width 0.25) (layer B.Cu) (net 3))
 (segment (start 161.76 95.24) (end 161.76 96.1) (width 0.25) (layer B.Cu) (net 3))
 (segment (start 163.1 93.9) (end 161.76 95.24) (width 0.25) (layer B.Cu) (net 3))
 (segment (start 164.1 93.9) (end 163.1 93.9) (width 0.25) (layer B.Cu) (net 3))
 (segment (start 165.45 92.52) (end 165.45 92.55) (width 0.25) (layer B.Cu) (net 3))
 (segment (start 165.45 92.55) (end 164.1 93.9) (width 0.25) (layer B.Cu) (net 3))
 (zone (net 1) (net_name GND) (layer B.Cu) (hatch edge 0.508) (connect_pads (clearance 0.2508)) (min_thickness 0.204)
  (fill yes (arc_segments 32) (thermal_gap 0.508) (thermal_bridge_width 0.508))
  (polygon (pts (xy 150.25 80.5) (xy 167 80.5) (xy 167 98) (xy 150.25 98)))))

